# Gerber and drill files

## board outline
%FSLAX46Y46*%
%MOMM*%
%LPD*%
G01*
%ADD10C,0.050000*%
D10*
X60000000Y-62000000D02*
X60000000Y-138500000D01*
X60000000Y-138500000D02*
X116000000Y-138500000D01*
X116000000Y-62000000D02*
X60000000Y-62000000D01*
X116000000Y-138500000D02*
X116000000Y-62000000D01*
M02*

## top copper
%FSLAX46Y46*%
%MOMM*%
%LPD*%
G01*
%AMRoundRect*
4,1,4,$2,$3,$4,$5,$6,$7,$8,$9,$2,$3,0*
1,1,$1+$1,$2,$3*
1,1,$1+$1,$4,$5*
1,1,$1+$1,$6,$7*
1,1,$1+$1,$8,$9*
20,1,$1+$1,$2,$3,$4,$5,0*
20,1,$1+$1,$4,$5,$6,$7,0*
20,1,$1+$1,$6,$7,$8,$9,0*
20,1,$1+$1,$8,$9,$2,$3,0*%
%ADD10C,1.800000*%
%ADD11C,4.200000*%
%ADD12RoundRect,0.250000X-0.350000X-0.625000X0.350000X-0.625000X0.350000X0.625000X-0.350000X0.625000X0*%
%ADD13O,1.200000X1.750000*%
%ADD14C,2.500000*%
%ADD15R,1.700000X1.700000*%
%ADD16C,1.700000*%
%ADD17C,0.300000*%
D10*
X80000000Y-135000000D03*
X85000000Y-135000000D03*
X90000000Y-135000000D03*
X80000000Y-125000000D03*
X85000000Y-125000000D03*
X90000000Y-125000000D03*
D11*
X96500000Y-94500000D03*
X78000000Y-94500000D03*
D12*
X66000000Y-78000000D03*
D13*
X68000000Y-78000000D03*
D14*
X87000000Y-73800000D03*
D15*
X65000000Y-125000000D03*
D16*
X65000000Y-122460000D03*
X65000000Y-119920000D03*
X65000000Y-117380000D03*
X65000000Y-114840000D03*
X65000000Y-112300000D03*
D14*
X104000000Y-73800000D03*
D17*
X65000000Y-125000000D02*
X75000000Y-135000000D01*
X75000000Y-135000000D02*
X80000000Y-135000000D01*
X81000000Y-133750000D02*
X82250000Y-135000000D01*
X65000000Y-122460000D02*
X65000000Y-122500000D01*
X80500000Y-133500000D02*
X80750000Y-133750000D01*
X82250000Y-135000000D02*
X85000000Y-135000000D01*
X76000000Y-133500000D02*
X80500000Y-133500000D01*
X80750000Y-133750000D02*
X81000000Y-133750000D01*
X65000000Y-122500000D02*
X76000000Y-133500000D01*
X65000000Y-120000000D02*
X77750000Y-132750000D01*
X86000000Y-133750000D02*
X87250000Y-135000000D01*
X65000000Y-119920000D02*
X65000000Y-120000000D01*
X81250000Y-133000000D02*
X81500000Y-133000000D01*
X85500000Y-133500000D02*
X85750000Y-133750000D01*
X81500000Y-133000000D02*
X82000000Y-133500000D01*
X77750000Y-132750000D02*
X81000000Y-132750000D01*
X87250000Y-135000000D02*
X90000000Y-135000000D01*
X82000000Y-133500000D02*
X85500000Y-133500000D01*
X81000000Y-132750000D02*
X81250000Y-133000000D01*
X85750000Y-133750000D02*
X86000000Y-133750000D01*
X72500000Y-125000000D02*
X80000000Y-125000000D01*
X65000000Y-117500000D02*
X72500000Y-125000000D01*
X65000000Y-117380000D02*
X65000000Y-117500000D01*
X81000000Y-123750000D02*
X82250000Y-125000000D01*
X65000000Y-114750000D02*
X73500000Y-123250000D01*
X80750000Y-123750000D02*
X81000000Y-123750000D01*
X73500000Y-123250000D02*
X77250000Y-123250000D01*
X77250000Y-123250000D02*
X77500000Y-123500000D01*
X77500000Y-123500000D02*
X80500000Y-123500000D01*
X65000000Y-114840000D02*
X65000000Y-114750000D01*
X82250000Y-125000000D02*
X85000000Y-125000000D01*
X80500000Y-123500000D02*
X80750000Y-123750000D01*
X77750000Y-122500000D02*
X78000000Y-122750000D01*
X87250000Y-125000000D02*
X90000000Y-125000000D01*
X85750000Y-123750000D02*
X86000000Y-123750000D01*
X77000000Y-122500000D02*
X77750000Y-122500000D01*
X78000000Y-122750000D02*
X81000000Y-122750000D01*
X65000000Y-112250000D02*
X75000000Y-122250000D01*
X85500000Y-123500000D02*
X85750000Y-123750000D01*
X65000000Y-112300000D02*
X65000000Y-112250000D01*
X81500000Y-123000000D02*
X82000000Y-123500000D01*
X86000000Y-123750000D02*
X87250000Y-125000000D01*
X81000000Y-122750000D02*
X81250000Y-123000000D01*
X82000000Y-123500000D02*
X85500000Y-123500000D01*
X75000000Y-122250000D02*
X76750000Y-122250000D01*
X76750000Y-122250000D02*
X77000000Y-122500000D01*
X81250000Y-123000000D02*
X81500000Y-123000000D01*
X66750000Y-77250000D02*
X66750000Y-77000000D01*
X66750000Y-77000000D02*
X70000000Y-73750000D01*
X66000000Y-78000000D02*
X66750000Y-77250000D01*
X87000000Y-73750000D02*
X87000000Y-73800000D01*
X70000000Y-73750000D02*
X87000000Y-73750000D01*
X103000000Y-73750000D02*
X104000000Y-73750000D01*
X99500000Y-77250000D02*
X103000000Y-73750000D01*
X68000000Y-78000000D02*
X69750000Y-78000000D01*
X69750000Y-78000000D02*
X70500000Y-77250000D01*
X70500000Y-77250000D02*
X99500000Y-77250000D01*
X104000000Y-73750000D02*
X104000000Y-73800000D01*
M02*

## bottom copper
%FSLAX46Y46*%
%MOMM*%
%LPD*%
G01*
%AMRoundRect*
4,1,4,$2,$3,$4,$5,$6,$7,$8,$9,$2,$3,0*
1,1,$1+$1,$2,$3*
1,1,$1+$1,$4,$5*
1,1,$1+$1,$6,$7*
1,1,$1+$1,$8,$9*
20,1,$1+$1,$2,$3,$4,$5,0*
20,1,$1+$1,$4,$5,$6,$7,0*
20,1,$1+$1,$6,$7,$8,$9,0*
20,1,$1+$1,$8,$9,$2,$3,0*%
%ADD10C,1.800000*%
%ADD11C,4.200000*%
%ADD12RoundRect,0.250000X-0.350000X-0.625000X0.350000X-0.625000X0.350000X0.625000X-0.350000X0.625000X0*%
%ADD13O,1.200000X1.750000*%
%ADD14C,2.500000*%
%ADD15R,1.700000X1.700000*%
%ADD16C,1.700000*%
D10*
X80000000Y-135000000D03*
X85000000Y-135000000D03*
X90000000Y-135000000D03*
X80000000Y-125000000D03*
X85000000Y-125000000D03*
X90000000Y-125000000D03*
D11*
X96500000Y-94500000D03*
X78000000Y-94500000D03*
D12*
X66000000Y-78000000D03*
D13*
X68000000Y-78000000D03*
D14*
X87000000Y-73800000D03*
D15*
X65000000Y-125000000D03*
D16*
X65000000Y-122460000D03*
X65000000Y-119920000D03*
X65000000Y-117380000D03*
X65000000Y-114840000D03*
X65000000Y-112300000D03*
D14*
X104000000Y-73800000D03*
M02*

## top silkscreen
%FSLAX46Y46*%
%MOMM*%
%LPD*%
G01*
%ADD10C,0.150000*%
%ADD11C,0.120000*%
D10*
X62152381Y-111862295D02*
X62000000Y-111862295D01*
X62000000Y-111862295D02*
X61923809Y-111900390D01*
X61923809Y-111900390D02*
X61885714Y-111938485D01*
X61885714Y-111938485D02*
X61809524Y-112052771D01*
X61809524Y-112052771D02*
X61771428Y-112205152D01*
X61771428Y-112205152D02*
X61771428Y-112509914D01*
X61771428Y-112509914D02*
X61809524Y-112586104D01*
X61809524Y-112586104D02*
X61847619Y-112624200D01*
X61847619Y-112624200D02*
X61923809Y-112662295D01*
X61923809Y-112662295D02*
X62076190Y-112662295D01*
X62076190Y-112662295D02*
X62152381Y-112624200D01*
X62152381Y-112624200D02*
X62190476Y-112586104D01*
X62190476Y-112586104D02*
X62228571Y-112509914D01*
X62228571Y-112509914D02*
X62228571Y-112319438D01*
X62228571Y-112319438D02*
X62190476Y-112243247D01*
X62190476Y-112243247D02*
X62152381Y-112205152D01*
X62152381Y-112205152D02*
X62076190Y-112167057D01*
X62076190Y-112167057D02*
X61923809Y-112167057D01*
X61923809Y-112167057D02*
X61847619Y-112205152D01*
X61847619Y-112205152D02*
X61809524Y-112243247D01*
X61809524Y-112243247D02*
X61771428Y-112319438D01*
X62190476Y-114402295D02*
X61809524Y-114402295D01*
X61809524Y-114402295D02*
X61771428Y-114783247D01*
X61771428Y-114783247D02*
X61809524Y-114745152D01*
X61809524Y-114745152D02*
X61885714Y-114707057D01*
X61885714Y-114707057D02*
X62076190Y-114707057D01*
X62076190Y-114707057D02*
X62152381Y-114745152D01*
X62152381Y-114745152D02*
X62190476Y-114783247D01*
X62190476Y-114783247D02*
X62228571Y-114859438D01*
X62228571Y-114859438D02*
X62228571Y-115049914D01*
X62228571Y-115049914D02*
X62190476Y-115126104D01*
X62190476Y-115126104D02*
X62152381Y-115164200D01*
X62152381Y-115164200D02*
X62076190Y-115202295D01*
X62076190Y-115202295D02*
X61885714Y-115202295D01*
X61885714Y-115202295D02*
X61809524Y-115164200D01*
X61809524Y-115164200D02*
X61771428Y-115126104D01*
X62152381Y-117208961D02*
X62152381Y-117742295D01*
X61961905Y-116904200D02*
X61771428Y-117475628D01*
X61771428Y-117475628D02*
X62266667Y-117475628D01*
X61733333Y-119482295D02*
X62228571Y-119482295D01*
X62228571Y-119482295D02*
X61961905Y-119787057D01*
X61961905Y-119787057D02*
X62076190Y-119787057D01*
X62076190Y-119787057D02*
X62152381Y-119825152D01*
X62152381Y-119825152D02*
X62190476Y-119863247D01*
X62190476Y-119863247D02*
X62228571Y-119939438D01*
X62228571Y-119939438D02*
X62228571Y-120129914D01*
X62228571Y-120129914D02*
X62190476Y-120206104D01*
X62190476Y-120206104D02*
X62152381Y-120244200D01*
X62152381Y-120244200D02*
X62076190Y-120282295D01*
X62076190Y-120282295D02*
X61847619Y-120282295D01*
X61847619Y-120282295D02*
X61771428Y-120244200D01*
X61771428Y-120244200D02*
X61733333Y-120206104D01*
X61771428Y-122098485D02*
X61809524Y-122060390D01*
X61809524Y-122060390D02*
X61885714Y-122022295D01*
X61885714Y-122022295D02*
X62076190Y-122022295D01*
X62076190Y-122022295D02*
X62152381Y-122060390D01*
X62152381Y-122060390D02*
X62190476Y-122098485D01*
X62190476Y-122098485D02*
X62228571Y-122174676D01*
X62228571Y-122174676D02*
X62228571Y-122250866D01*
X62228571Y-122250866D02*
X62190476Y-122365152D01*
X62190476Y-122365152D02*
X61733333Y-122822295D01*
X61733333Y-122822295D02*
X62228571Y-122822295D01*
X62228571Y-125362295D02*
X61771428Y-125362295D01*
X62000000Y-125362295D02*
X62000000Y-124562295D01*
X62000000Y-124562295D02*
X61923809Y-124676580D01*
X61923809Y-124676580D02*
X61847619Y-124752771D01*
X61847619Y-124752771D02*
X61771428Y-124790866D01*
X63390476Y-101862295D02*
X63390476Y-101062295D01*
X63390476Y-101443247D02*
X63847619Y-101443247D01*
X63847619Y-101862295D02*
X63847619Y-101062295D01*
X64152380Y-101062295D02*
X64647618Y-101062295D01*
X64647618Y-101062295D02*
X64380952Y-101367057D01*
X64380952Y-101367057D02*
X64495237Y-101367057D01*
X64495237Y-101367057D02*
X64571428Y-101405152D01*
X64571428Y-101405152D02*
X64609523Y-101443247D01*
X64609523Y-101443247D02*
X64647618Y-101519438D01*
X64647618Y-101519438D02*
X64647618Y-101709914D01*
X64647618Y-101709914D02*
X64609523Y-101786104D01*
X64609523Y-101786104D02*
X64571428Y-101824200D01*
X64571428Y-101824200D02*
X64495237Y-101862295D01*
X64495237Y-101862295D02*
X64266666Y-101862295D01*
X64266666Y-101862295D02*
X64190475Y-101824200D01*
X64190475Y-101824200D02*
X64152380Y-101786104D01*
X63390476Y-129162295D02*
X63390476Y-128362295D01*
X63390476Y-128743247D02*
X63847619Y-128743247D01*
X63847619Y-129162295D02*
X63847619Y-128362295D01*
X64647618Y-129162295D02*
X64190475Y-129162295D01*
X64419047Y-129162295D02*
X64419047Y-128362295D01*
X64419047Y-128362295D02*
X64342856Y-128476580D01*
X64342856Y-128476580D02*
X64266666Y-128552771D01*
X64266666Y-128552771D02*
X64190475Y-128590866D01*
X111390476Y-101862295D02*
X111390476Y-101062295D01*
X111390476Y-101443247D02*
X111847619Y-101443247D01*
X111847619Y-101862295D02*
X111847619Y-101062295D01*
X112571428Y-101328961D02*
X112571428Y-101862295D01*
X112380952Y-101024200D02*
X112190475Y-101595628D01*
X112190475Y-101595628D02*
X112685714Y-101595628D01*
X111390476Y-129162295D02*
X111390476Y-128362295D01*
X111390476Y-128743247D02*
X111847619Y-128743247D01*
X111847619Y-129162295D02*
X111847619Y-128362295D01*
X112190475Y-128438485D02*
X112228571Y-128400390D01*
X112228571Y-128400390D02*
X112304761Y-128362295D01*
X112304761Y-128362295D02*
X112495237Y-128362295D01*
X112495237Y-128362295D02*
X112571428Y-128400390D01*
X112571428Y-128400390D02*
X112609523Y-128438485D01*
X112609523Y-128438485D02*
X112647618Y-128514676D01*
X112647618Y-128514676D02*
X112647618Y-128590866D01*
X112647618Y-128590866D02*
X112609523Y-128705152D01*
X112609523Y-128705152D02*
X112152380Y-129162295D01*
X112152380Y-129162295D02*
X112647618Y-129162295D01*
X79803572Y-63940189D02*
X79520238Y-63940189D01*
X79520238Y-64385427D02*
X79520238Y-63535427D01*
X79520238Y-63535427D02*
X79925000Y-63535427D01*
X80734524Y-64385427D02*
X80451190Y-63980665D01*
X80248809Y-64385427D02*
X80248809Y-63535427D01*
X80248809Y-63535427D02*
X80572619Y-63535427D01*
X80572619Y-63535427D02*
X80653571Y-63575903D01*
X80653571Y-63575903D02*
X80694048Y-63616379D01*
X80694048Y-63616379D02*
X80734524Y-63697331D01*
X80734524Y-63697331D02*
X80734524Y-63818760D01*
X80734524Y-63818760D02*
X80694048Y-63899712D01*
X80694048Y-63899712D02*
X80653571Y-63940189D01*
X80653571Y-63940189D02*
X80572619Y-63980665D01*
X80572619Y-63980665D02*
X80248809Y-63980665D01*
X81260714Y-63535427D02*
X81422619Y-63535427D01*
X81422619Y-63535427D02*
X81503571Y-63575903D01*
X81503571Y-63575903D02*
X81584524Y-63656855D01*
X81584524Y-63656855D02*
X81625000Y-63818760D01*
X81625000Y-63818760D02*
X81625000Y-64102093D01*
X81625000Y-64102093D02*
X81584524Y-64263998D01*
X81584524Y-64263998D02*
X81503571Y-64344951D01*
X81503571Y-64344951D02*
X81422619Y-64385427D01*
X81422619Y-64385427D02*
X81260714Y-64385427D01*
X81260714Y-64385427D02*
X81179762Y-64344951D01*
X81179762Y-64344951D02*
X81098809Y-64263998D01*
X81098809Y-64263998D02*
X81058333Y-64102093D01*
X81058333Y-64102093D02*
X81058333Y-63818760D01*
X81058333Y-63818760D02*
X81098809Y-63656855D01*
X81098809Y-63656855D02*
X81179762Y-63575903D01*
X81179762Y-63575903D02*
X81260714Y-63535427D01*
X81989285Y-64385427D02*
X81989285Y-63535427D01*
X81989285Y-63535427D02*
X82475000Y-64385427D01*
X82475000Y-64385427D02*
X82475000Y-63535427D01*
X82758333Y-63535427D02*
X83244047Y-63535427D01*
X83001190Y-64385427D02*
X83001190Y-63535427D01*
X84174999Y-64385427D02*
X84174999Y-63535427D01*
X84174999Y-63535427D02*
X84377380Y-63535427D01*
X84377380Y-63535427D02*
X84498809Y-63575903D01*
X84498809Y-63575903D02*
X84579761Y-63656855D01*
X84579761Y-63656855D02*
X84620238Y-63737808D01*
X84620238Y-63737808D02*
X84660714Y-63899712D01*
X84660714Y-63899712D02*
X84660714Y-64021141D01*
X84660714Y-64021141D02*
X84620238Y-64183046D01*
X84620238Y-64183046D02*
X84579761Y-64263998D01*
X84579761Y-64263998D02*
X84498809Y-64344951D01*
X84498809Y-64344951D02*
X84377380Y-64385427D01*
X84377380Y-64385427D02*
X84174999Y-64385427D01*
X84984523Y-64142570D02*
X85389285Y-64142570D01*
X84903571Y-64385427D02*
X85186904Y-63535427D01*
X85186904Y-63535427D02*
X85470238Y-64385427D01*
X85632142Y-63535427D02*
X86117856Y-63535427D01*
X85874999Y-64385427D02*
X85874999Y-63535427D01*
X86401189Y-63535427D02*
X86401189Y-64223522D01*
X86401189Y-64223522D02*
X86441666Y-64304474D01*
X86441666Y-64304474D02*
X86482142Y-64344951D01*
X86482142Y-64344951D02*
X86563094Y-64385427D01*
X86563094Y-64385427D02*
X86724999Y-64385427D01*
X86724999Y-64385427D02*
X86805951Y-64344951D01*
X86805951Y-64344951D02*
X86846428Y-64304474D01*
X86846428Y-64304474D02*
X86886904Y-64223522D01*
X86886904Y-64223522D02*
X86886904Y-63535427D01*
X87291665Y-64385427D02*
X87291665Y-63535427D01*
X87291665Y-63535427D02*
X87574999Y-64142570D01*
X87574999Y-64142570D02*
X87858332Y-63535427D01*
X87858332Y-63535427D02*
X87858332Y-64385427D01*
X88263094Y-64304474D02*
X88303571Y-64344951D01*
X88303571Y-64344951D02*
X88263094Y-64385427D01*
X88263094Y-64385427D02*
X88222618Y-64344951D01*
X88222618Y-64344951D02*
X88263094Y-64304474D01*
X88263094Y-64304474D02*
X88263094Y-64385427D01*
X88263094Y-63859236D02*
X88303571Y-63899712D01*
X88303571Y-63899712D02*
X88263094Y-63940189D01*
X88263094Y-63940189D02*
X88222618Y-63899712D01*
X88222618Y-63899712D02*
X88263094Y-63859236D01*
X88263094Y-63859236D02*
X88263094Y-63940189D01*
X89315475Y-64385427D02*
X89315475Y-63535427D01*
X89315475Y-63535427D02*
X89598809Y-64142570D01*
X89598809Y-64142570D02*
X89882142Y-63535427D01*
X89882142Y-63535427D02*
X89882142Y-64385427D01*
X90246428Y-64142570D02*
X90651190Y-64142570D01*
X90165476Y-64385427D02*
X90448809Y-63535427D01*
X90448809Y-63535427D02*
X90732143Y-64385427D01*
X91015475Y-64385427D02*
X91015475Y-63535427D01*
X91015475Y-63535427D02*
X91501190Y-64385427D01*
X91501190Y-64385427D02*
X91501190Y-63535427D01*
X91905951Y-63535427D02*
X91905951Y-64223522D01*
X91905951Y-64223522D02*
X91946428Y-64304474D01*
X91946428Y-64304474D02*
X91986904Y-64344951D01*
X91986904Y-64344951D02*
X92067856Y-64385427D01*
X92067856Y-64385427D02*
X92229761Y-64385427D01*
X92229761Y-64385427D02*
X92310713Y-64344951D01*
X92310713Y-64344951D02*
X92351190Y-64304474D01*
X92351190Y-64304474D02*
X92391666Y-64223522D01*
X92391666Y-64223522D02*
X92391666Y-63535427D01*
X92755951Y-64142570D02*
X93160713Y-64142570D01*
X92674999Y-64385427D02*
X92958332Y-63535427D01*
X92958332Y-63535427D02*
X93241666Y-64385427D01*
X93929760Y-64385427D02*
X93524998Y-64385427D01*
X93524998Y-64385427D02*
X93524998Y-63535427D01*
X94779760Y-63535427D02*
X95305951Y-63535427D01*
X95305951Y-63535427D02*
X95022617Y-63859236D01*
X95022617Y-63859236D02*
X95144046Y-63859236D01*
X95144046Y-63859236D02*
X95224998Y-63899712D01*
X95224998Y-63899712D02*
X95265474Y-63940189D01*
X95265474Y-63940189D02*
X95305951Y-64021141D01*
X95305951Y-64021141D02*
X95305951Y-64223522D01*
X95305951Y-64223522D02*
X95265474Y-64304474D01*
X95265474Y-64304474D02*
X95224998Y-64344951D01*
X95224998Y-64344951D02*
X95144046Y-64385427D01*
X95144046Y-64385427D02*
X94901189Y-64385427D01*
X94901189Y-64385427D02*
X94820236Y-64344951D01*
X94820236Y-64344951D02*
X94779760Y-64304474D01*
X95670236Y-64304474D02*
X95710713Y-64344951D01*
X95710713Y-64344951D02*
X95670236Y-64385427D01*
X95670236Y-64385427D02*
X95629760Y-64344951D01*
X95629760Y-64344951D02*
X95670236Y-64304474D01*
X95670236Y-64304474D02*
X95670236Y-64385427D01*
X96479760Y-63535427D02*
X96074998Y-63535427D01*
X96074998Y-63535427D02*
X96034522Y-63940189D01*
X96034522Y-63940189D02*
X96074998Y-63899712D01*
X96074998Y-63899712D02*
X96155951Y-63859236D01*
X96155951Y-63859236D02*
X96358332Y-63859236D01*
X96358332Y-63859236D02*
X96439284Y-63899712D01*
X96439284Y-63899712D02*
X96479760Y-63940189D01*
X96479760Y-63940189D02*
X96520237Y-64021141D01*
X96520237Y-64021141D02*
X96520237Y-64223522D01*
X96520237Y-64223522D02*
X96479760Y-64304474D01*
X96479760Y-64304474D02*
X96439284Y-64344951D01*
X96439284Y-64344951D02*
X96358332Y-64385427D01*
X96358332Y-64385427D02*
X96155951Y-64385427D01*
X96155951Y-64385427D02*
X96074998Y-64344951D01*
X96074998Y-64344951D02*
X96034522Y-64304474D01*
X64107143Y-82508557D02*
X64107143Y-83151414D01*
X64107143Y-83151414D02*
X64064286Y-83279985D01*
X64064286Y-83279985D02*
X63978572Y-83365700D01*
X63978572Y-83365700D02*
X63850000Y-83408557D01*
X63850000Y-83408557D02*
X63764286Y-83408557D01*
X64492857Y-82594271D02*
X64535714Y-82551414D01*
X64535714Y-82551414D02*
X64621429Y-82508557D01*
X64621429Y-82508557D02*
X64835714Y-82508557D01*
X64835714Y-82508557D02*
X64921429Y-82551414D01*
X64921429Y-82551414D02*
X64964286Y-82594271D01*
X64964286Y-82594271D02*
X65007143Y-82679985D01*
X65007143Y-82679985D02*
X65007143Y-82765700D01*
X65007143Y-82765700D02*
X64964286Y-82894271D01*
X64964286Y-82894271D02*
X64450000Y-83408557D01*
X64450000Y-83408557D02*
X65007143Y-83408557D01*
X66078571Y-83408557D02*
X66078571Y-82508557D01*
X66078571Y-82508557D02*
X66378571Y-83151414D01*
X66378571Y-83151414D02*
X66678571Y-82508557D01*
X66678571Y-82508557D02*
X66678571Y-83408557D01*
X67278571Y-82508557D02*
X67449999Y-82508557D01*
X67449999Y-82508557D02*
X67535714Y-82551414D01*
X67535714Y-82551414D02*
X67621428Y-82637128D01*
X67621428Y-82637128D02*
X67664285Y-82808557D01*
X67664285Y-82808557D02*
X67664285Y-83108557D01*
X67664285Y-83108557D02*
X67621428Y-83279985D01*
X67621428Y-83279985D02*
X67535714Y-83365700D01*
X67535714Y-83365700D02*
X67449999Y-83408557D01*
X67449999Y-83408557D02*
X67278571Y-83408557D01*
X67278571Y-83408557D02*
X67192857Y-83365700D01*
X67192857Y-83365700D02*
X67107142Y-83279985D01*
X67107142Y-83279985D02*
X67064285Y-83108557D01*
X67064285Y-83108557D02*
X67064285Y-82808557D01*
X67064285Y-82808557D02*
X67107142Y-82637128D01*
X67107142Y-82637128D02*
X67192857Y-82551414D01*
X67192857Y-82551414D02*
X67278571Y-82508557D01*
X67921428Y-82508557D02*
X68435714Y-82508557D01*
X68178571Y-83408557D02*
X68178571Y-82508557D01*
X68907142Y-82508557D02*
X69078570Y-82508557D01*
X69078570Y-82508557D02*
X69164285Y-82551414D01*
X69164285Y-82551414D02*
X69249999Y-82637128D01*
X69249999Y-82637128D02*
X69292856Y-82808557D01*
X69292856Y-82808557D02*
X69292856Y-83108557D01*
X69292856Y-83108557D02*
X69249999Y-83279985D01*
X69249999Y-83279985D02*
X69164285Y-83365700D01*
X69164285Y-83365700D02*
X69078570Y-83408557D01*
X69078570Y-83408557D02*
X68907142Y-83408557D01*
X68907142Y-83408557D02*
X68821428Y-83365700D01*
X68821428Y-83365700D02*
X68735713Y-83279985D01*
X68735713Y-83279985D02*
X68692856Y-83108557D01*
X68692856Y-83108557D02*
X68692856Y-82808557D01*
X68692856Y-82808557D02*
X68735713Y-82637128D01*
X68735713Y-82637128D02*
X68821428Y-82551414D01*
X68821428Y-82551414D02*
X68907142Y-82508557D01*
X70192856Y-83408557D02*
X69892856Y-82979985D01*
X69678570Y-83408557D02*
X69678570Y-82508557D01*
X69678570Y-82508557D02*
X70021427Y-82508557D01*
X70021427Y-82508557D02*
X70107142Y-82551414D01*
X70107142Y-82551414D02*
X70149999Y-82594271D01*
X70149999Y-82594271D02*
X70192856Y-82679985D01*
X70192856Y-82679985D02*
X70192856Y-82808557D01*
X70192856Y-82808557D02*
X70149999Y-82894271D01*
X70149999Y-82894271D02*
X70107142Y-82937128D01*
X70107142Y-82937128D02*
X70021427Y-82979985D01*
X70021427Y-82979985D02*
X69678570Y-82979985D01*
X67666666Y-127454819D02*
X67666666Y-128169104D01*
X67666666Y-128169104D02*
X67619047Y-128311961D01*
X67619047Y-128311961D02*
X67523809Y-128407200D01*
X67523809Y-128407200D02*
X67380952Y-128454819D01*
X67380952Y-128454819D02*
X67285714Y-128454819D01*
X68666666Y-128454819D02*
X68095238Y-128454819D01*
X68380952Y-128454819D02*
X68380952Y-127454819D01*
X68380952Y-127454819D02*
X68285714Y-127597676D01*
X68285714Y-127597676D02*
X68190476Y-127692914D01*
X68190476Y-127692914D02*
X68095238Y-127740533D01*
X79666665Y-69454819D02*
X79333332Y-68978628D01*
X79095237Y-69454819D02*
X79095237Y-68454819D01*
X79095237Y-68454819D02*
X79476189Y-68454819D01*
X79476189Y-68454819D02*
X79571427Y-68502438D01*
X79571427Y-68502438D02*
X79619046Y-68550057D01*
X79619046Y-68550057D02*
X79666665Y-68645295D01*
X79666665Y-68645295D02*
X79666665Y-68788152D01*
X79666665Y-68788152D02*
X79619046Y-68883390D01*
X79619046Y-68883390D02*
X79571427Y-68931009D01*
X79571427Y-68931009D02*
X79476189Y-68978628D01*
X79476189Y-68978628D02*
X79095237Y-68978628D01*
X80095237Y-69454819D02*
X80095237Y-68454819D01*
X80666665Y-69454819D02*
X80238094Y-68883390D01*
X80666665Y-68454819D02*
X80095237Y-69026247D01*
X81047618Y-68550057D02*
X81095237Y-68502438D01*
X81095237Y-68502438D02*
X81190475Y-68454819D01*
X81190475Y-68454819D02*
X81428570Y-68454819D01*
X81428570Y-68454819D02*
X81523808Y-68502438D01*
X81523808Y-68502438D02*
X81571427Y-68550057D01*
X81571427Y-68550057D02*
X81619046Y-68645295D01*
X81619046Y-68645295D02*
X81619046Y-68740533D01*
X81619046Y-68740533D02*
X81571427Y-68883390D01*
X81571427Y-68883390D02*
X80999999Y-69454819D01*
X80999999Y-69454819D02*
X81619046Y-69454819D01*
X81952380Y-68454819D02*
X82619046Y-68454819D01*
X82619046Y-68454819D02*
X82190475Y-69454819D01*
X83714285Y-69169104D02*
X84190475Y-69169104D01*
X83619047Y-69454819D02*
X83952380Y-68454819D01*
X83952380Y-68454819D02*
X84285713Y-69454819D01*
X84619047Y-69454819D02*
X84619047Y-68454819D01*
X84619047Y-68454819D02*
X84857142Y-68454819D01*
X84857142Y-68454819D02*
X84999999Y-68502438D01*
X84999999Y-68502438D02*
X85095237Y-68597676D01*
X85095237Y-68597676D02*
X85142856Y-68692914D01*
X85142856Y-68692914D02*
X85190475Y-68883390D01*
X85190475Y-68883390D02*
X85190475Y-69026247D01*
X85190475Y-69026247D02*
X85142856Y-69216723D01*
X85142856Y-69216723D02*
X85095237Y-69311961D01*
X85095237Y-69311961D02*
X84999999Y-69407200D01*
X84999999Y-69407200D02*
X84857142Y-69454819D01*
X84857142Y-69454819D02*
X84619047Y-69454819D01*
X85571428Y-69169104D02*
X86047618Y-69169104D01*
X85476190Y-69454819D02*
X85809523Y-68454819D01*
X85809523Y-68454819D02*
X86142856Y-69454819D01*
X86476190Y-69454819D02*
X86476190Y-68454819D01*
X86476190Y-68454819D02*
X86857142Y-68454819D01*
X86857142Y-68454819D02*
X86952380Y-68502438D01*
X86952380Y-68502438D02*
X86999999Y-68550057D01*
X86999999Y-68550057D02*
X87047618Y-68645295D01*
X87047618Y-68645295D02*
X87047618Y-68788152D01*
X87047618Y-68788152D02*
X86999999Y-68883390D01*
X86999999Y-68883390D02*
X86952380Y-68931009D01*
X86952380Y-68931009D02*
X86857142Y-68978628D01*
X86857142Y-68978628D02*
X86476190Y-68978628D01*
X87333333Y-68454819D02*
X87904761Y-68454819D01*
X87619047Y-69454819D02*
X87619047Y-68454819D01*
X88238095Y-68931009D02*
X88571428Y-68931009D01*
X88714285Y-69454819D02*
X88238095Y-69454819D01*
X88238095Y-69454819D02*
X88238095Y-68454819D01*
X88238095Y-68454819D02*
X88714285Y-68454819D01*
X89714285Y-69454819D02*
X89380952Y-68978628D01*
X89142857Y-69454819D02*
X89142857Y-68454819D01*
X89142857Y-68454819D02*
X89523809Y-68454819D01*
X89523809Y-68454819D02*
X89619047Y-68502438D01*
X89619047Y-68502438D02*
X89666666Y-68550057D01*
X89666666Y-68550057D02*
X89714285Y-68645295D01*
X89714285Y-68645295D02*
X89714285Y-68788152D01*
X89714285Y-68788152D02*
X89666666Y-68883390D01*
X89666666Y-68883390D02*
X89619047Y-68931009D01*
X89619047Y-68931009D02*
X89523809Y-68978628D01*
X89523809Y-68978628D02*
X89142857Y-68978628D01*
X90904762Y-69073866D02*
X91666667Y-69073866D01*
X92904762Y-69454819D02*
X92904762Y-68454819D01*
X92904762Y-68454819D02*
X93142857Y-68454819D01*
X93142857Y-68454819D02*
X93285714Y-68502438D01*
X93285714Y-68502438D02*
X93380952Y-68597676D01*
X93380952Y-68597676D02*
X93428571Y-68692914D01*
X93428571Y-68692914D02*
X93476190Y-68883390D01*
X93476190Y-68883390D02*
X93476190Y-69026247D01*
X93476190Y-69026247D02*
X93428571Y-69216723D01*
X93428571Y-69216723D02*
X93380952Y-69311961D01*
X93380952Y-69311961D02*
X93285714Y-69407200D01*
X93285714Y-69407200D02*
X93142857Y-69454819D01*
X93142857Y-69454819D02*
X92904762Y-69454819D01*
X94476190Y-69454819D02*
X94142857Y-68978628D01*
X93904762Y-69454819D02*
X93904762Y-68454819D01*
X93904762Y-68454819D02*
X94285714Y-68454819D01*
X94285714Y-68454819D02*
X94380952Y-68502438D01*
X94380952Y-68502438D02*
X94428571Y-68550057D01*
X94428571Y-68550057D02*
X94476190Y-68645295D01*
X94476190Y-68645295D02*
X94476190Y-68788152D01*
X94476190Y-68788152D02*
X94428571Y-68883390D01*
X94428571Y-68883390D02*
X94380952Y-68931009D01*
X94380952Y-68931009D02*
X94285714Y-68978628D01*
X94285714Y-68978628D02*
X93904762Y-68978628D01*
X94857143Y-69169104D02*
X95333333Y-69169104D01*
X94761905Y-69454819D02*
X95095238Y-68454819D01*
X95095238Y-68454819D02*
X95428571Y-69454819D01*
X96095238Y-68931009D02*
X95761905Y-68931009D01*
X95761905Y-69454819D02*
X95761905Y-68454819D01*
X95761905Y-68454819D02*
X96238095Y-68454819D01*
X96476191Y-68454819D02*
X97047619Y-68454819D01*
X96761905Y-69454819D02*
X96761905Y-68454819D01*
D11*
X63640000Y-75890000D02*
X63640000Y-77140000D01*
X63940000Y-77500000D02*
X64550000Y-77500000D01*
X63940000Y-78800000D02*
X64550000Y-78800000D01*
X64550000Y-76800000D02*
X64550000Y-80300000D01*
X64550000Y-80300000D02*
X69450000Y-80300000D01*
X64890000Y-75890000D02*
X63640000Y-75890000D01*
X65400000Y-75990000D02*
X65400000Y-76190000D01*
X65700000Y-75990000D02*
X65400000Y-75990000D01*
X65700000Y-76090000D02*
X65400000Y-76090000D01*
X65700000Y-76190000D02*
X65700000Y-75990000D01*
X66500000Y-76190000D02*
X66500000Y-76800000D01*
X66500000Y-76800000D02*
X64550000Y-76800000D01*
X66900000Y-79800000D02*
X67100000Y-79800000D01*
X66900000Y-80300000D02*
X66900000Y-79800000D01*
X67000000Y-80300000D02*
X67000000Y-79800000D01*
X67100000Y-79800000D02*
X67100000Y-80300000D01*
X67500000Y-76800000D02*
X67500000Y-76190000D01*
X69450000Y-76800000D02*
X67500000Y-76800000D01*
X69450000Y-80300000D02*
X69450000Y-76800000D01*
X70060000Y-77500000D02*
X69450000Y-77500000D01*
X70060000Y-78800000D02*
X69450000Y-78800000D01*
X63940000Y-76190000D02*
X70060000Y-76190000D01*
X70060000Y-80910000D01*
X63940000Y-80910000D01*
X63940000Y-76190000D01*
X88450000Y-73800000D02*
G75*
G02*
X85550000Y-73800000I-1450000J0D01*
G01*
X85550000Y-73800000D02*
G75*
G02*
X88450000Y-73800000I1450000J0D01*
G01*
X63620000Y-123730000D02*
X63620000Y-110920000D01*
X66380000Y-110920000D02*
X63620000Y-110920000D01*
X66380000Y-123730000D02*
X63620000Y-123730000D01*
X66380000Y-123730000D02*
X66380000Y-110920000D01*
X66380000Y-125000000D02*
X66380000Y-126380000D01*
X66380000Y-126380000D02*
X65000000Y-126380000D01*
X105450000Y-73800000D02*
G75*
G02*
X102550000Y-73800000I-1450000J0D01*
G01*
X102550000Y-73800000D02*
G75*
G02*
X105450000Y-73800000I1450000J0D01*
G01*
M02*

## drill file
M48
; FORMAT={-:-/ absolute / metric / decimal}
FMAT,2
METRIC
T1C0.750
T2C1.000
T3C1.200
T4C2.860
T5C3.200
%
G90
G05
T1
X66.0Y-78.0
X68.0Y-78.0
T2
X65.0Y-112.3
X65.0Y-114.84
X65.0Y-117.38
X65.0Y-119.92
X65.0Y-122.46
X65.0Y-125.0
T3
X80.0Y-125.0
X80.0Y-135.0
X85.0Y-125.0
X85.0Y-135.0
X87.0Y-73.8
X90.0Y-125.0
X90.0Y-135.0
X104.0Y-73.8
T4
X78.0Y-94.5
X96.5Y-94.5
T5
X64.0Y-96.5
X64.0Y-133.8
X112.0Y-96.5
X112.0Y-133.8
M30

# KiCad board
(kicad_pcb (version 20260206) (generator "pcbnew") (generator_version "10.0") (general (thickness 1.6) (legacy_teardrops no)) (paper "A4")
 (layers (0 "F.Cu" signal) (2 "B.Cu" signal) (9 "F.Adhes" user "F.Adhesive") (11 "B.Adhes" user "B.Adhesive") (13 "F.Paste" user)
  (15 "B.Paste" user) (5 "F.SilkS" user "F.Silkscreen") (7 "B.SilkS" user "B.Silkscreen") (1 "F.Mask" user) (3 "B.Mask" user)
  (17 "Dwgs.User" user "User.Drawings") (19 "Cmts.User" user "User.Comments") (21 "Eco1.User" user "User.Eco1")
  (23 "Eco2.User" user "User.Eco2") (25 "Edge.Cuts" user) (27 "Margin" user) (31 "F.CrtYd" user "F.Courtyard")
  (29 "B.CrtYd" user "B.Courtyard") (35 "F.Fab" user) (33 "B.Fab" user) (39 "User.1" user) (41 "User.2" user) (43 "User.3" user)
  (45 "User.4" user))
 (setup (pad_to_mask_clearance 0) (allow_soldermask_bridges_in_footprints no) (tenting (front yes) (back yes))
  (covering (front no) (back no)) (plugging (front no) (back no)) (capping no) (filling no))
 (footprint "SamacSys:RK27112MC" (layer "F.Cu") (at 85 94.5 -90)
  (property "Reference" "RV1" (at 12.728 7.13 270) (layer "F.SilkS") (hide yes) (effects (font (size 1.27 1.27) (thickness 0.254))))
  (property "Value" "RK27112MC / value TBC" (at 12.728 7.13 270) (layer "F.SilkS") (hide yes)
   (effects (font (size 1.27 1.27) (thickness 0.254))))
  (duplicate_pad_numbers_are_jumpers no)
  (pad "1" thru_hole circle (at 40.5 5 270) (size 1.8 1.8) (drill 1.2) (layers "*.Cu" "*.Mask") (remove_unused_layers no) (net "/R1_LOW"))
  (pad "2" thru_hole circle (at 40.5 0 270) (size 1.8 1.8) (drill 1.2) (layers "*.Cu" "*.Mask") (remove_unused_layers no) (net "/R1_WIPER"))
  (pad "3" thru_hole circle (at 40.5 -5 270) (size 1.8 1.8) (drill 1.2) (layers "*.Cu" "*.Mask") (remove_unused_layers no) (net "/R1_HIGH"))
  (pad "4" thru_hole circle (at 30.5 5 270) (size 1.8 1.8) (drill 1.2) (layers "*.Cu" "*.Mask") (remove_unused_layers no) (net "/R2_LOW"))
  (pad "5" thru_hole circle (at 30.5 0 270) (size 1.8 1.8) (drill 1.2) (layers "*.Cu" "*.Mask") (remove_unused_layers no) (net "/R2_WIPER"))
  (pad "6" thru_hole circle (at 30.5 -5 270) (size 1.8 1.8) (drill 1.2) (layers "*.Cu" "*.Mask") (remove_unused_layers no) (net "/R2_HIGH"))
  (pad "7" thru_hole circle (at 0 -11.5 270) (size 4.2 4.2) (drill 2.86) (layers "*.Cu" "*.Mask") (remove_unused_layers no)
   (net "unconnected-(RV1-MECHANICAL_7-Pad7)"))
  (pad "8" thru_hole circle (at 0 7 270) (size 4.2 4.2) (drill 2.86) (layers "*.Cu" "*.Mask") (remove_unused_layers no)
   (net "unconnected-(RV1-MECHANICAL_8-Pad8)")))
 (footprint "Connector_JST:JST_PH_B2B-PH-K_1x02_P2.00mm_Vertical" (layer "F.Cu") (at 66 78)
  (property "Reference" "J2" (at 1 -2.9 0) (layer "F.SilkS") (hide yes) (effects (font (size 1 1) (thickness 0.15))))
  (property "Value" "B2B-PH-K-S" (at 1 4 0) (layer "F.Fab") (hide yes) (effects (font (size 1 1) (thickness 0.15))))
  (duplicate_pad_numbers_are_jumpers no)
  (fp_line (start -2.36 -2.11) (end -2.36 -0.86) (stroke (width 0.12) (type solid)) (layer "F.SilkS"))
  (fp_line (start -2.06 -0.5) (end -1.45 -0.5) (stroke (width 0.12) (type solid)) (layer "F.SilkS"))
  (fp_line (start -2.06 0.8) (end -1.45 0.8) (stroke (width 0.12) (type solid)) (layer "F.SilkS"))
  (fp_line (start -1.45 -1.2) (end -1.45 2.3) (stroke (width 0.12) (type solid)) (layer "F.SilkS"))
  (fp_line (start -1.45 2.3) (end 3.45 2.3) (stroke (width 0.12) (type solid)) (layer "F.SilkS"))
  (fp_line (start -1.11 -2.11) (end -2.36 -2.11) (stroke (width 0.12) (type solid)) (layer "F.SilkS"))
  (fp_line (start -0.6 -2.01) (end -0.6 -1.81) (stroke (width 0.12) (type solid)) (layer "F.SilkS"))
  (fp_line (start -0.3 -2.01) (end -0.6 -2.01) (stroke (width 0.12) (type solid)) (layer "F.SilkS"))
  (fp_line (start -0.3 -1.91) (end -0.6 -1.91) (stroke (width 0.12) (type solid)) (layer "F.SilkS"))
  (fp_line (start -0.3 -1.81) (end -0.3 -2.01) (stroke (width 0.12) (type solid)) (layer "F.SilkS"))
  (fp_line (start 0.5 -1.81) (end 0.5 -1.2) (stroke (width 0.12) (type solid)) (layer "F.SilkS"))
  (fp_line (start 0.5 -1.2) (end -1.45 -1.2) (stroke (width 0.12) (type solid)) (layer "F.SilkS"))
  (fp_line (start 0.9 1.8) (end 1.1 1.8) (stroke (width 0.12) (type solid)) (layer "F.SilkS"))
  (fp_line (start 0.9 2.3) (end 0.9 1.8) (stroke (width 0.12) (type solid)) (layer "F.SilkS"))
  (fp_line (start 1 2.3) (end 1 1.8) (stroke (width 0.12) (type solid)) (layer "F.SilkS"))
  (fp_line (start 1.1 1.8) (end 1.1 2.3) (stroke (width 0.12) (type solid)) (layer "F.SilkS"))
  (fp_line (start 1.5 -1.2) (end 1.5 -1.81) (stroke (width 0.12) (type solid)) (layer "F.SilkS"))
  (fp_line (start 3.45 -1.2) (end 1.5 -1.2) (stroke (width 0.12) (type solid)) (layer "F.SilkS"))
  (fp_line (start 3.45 2.3) (end 3.45 -1.2) (stroke (width 0.12) (type solid)) (layer "F.SilkS"))
  (fp_line (start 4.06 -0.5) (end 3.45 -0.5) (stroke (width 0.12) (type solid)) (layer "F.SilkS"))
  (fp_line (start 4.06 0.8) (end 3.45 0.8) (stroke (width 0.12) (type solid)) (layer "F.SilkS"))
  (fp_rect (start -2.06 -1.81) (end 4.06 2.91) (stroke (width 0.12) (type solid)) (fill no) (layer "F.SilkS"))
  (pad "1" thru_hole roundrect (at 0 0) (size 1.2 1.75) (drill 0.75) (layers "*.Cu" "*.Mask") (remove_unused_layers no)
   (roundrect_rratio 0.208333) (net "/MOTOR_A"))
  (pad "2" thru_hole oval (at 2 0) (size 1.2 1.75) (drill 0.75) (layers "*.Cu" "*.Mask") (remove_unused_layers no) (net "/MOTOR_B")))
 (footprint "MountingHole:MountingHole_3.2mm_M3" (layer "F.Cu") (at 112 133.8)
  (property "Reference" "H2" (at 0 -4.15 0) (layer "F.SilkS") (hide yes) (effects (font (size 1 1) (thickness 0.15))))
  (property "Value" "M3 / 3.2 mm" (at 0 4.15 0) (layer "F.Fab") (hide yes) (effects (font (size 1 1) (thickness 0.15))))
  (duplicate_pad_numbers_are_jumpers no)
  (pad "" np_thru_hole circle (at 0 0) (size 3.2 3.2) (drill 3.2) (layers "*.Cu" "*.Mask")))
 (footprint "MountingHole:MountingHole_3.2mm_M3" (layer "F.Cu") (at 64 96.5)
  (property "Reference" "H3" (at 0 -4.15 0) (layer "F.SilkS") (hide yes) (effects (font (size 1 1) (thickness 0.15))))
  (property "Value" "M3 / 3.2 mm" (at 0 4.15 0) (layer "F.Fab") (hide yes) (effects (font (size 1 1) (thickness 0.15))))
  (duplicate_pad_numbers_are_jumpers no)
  (pad "" np_thru_hole circle (at 0 0) (size 3.2 3.2) (drill 3.2) (layers "*.Cu" "*.Mask")))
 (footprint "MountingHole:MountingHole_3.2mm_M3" (layer "F.Cu") (at 64 133.8)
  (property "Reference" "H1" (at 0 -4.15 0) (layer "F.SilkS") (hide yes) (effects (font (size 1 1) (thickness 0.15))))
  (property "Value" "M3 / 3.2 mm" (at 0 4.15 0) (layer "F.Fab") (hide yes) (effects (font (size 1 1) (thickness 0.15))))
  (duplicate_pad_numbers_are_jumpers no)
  (pad "" np_thru_hole circle (at 0 0) (size 3.2 3.2) (drill 3.2) (layers "*.Cu" "*.Mask")))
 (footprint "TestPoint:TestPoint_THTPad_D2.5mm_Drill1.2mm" (layer "F.Cu") (at 87 73.8)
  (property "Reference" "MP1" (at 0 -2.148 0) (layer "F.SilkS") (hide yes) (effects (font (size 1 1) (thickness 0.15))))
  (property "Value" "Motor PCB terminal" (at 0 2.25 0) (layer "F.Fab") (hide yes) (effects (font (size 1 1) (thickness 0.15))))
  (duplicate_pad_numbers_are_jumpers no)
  (fp_circle (center 0 0) (end 0 1.45) (stroke (width 0.12) (type solid)) (fill no) (layer "F.SilkS"))
  (pad "1" thru_hole circle (at 0 0) (size 2.5 2.5) (drill 1.2) (layers "*.Cu" "*.Mask") (remove_unused_layers no) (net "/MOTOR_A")))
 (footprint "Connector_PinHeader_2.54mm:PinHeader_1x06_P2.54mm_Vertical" (layer "F.Cu") (at 65 125 180)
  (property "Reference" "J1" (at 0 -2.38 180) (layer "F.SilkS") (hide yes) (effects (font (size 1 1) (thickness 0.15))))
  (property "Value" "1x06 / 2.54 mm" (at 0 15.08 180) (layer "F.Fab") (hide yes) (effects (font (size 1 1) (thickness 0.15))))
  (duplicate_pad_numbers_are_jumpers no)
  (fp_line (start 1.38 1.27) (end 1.38 14.08) (stroke (width 0.12) (type solid)) (layer "F.SilkS"))
  (fp_line (start -1.38 14.08) (end 1.38 14.08) (stroke (width 0.12) (type solid)) (layer "F.SilkS"))
  (fp_line (start -1.38 1.27) (end 1.38 1.27) (stroke (width 0.12) (type solid)) (layer "F.SilkS"))
  (fp_line (start -1.38 1.27) (end -1.38 14.08) (stroke (width 0.12) (type solid)) (layer "F.SilkS"))
  (fp_line (start -1.38 0) (end -1.38 -1.38) (stroke (width 0.12) (type solid)) (layer "F.SilkS"))
  (fp_line (start -1.38 -1.38) (end 0 -1.38) (stroke (width 0.12) (type solid)) (layer "F.SilkS"))
  (pad "1" thru_hole rect (at 0 0 180) (size 1.7 1.7) (drill 1) (layers "*.Cu" "*.Mask") (remove_unused_layers no) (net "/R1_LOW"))
  (pad "2" thru_hole circle (at 0 2.54 180) (size 1.7 1.7) (drill 1) (layers "*.Cu" "*.Mask") (remove_unused_layers no) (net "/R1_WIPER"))
  (pad "3" thru_hole circle (at 0 5.08 180) (size 1.7 1.7) (drill 1) (layers "*.Cu" "*.Mask") (remove_unused_layers no) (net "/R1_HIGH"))
  (pad "4" thru_hole circle (at 0 7.62 180) (size 1.7 1.7) (drill 1) (layers "*.Cu" "*.Mask") (remove_unused_layers no) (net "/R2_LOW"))
  (pad "5" thru_hole circle (at 0 10.16 180) (size 1.7 1.7) (drill 1) (layers "*.Cu" "*.Mask") (remove_unused_layers no) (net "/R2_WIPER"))
  (pad "6" thru_hole circle (at 0 12.7 180) (size 1.7 1.7) (drill 1) (layers "*.Cu" "*.Mask") (remove_unused_layers no) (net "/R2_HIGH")))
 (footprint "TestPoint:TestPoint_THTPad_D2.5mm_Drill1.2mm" (layer "F.Cu") (at 104 73.8)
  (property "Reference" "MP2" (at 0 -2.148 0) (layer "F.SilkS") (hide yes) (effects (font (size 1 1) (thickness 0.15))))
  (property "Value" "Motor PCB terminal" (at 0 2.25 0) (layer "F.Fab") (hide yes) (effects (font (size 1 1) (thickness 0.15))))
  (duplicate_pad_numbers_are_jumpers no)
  (fp_circle (center 0 0) (end 0 1.45) (stroke (width 0.12) (type solid)) (fill no) (layer "F.SilkS"))
  (pad "1" thru_hole circle (at 0 0) (size 2.5 2.5) (drill 1.2) (layers "*.Cu" "*.Mask") (remove_unused_layers no) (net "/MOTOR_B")))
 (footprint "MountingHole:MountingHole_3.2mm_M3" (layer "F.Cu") (at 112 96.5)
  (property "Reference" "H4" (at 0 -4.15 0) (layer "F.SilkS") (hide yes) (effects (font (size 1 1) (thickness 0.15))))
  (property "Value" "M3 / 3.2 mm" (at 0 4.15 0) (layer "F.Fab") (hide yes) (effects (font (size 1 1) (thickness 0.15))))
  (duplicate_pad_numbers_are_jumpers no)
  (pad "" np_thru_hole circle (at 0 0) (size 3.2 3.2) (drill 3.2) (layers "*.Cu" "*.Mask")))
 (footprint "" (layer "F.Cu") (at 85 140)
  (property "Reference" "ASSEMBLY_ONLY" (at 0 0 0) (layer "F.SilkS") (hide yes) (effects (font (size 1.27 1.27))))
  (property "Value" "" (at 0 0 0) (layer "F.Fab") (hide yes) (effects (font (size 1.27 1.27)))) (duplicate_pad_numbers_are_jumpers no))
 (gr_line (start 60 62) (end 60 138.5) (stroke (width 0.05) (type default)) (layer "Edge.Cuts"))
 (gr_line (start 60 138.5) (end 116 138.5) (stroke (width 0.05) (type default)) (layer "Edge.Cuts"))
 (gr_line (start 116 62) (end 60 62) (stroke (width 0.05) (type default)) (layer "Edge.Cuts"))
 (gr_line (start 116 138.5) (end 116 62) (stroke (width 0.05) (type default)) (layer "Edge.Cuts"))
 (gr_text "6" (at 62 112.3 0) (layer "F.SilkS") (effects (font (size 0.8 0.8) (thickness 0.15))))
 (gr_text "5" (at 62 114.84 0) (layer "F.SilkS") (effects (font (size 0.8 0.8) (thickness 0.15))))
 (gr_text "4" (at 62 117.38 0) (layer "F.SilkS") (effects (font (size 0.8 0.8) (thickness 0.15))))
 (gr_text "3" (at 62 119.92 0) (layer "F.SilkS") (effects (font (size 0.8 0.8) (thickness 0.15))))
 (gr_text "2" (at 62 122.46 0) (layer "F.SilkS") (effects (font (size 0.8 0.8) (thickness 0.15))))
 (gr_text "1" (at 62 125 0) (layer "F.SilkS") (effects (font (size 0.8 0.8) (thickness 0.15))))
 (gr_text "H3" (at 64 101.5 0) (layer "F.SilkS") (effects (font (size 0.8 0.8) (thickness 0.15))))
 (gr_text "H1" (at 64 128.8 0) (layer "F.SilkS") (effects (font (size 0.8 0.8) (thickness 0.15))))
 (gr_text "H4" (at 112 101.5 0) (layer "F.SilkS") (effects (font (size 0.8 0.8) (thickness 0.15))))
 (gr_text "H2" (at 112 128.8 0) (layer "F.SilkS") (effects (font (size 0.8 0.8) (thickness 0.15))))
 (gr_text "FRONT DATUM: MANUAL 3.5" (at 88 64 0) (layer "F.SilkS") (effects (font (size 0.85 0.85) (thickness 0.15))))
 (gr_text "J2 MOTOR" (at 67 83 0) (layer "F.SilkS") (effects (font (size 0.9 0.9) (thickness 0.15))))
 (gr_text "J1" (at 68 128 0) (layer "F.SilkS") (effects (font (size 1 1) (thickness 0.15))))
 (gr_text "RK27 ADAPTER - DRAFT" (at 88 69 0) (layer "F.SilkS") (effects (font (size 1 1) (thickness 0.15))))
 (segment (start 65 125) (end 75 135) (width 0.3) (layer "F.Cu") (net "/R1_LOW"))
 (segment (start 75 135) (end 80 135) (width 0.3) (layer "F.Cu") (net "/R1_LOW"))
 (segment (start 81 133.75) (end 82.25 135) (width 0.3) (layer "F.Cu") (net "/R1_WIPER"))
 (segment (start 65 122.46) (end 65 122.5) (width 0.3) (layer "F.Cu") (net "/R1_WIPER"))
 (segment (start 80.5 133.5) (end 80.75 133.75) (width 0.3) (layer "F.Cu") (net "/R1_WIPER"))
 (segment (start 82.25 135) (end 85 135) (width 0.3) (layer "F.Cu") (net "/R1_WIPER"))
 (segment (start 76 133.5) (end 80.5 133.5) (width 0.3) (layer "F.Cu") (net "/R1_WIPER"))
 (segment (start 80.75 133.75) (end 81 133.75) (width 0.3) (layer "F.Cu") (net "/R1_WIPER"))
 (segment (start 65 122.5) (end 76 133.5) (width 0.3) (layer "F.Cu") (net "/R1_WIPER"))
 (segment (start 65 120) (end 77.75 132.75) (width 0.3) (layer "F.Cu") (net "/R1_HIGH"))
 (segment (start 86 133.75) (end 87.25 135) (width 0.3) (layer "F.Cu") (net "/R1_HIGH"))
 (segment (start 65 119.92) (end 65 120) (width 0.3) (layer "F.Cu") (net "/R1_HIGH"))
 (segment (start 81.25 133) (end 81.5 133) (width 0.3) (layer "F.Cu") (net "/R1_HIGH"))
 (segment (start 85.5 133.5) (end 85.75 133.75) (width 0.3) (layer "F.Cu") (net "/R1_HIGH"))
 (segment (start 81.5 133) (end 82 133.5) (width 0.3) (layer "F.Cu") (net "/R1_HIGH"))
 (segment (start 77.75 132.75) (end 81 132.75) (width 0.3) (layer "F.Cu") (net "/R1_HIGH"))
 (segment (start 87.25 135) (end 90 135) (width 0.3) (layer "F.Cu") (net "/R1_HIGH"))
 (segment (start 82 133.5) (end 85.5 133.5) (width 0.3) (layer "F.Cu") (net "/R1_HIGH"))
 (segment (start 81 132.75) (end 81.25 133) (width 0.3) (layer "F.Cu") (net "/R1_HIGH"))
 (segment (start 85.75 133.75) (end 86 133.75) (width 0.3) (layer "F.Cu") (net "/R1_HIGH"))
 (segment (start 72.5 125) (end 80 125) (width 0.3) (layer "F.Cu") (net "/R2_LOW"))
 (segment (start 65 117.5) (end 72.5 125) (width 0.3) (layer "F.Cu") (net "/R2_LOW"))
 (segment (start 65 117.38) (end 65 117.5) (width 0.3) (layer "F.Cu") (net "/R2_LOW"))
 (segment (start 81 123.75) (end 82.25 125) (width 0.3) (layer "F.Cu") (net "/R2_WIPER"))
 (segment (start 65 114.75) (end 73.5 123.25) (width 0.3) (layer "F.Cu") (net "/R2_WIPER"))
 (segment (start 80.75 123.75) (end 81 123.75) (width 0.3) (layer "F.Cu") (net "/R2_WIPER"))
 (segment (start 73.5 123.25) (end 77.25 123.25) (width 0.3) (layer "F.Cu") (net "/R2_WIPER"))
 (segment (start 77.25 123.25) (end 77.5 123.5) (width 0.3) (layer "F.Cu") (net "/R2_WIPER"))
 (segment (start 77.5 123.5) (end 80.5 123.5) (width 0.3) (layer "F.Cu") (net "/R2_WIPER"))
 (segment (start 65 114.84) (end 65 114.75) (width 0.3) (layer "F.Cu") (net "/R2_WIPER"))
 (segment (start 82.25 125) (end 85 125) (width 0.3) (layer "F.Cu") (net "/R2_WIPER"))
 (segment (start 80.5 123.5) (end 80.75 123.75) (width 0.3) (layer "F.Cu") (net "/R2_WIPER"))
 (segment (start 77.75 122.5) (end 78 122.75) (width 0.3) (layer "F.Cu") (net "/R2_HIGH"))
 (segment (start 87.25 125) (end 90 125) (width 0.3) (layer "F.Cu") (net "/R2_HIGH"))
 (segment (start 85.75 123.75) (end 86 123.75) (width 0.3) (layer "F.Cu") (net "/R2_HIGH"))
 (segment (start 77 122.5) (end 77.75 122.5) (width 0.3) (layer "F.Cu") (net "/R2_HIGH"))
 (segment (start 78 122.75) (end 81 122.75) (width 0.3) (layer "F.Cu") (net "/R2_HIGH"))
 (segment (start 65 112.25) (end 75 122.25) (width 0.3) (layer "F.Cu") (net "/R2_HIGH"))
 (segment (start 85.5 123.5) (end 85.75 123.75) (width 0.3) (layer "F.Cu") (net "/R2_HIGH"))
 (segment (start 65 112.3) (end 65 112.25) (width 0.3) (layer "F.Cu") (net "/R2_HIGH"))
 (segment (start 81.5 123) (end 82 123.5) (width 0.3) (layer "F.Cu") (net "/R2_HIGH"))
 (segment (start 86 123.75) (end 87.25 125) (width 0.3) (layer "F.Cu") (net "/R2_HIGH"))
 (segment (start 81 122.75) (end 81.25 123) (width 0.3) (layer "F.Cu") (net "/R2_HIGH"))
 (segment (start 82 123.5) (end 85.5 123.5) (width 0.3) (layer "F.Cu") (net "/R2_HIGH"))
 (segment (start 75 122.25) (end 76.75 122.25) (width 0.3) (layer "F.Cu") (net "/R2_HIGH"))
 (segment (start 76.75 122.25) (end 77 122.5) (width 0.3) (layer "F.Cu") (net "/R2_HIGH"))
 (segment (start 81.25 123) (end 81.5 123) (width 0.3) (layer "F.Cu") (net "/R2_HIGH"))
 (segment (start 66.75 77.25) (end 66.75 77) (width 0.3) (layer "F.Cu") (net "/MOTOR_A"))
 (segment (start 66.75 77) (end 70 73.75) (width 0.3) (layer "F.Cu") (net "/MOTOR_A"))
 (segment (start 66 78) (end 66.75 77.25) (width 0.3) (layer "F.Cu") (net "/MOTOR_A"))
 (segment (start 87 73.75) (end 87 73.8) (width 0.3) (layer "F.Cu") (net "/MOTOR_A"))
 (segment (start 70 73.75) (end 87 73.75) (width 0.3) (layer "F.Cu") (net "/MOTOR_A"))
 (segment (start 103 73.75) (end 104 73.75) (width 0.3) (layer "F.Cu") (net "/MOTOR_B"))
 (segment (start 99.5 77.25) (end 103 73.75) (width 0.3) (layer "F.Cu") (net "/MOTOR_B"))
 (segment (start 68 78) (end 69.75 78) (width 0.3) (layer "F.Cu") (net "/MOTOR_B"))
 (segment (start 69.75 78) (end 70.5 77.25) (width 0.3) (layer "F.Cu") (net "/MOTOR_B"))
 (segment (start 70.5 77.25) (end 99.5 77.25) (width 0.3) (layer "F.Cu") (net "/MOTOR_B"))
 (segment (start 104 73.75) (end 104 73.8) (width 0.3) (layer "F.Cu") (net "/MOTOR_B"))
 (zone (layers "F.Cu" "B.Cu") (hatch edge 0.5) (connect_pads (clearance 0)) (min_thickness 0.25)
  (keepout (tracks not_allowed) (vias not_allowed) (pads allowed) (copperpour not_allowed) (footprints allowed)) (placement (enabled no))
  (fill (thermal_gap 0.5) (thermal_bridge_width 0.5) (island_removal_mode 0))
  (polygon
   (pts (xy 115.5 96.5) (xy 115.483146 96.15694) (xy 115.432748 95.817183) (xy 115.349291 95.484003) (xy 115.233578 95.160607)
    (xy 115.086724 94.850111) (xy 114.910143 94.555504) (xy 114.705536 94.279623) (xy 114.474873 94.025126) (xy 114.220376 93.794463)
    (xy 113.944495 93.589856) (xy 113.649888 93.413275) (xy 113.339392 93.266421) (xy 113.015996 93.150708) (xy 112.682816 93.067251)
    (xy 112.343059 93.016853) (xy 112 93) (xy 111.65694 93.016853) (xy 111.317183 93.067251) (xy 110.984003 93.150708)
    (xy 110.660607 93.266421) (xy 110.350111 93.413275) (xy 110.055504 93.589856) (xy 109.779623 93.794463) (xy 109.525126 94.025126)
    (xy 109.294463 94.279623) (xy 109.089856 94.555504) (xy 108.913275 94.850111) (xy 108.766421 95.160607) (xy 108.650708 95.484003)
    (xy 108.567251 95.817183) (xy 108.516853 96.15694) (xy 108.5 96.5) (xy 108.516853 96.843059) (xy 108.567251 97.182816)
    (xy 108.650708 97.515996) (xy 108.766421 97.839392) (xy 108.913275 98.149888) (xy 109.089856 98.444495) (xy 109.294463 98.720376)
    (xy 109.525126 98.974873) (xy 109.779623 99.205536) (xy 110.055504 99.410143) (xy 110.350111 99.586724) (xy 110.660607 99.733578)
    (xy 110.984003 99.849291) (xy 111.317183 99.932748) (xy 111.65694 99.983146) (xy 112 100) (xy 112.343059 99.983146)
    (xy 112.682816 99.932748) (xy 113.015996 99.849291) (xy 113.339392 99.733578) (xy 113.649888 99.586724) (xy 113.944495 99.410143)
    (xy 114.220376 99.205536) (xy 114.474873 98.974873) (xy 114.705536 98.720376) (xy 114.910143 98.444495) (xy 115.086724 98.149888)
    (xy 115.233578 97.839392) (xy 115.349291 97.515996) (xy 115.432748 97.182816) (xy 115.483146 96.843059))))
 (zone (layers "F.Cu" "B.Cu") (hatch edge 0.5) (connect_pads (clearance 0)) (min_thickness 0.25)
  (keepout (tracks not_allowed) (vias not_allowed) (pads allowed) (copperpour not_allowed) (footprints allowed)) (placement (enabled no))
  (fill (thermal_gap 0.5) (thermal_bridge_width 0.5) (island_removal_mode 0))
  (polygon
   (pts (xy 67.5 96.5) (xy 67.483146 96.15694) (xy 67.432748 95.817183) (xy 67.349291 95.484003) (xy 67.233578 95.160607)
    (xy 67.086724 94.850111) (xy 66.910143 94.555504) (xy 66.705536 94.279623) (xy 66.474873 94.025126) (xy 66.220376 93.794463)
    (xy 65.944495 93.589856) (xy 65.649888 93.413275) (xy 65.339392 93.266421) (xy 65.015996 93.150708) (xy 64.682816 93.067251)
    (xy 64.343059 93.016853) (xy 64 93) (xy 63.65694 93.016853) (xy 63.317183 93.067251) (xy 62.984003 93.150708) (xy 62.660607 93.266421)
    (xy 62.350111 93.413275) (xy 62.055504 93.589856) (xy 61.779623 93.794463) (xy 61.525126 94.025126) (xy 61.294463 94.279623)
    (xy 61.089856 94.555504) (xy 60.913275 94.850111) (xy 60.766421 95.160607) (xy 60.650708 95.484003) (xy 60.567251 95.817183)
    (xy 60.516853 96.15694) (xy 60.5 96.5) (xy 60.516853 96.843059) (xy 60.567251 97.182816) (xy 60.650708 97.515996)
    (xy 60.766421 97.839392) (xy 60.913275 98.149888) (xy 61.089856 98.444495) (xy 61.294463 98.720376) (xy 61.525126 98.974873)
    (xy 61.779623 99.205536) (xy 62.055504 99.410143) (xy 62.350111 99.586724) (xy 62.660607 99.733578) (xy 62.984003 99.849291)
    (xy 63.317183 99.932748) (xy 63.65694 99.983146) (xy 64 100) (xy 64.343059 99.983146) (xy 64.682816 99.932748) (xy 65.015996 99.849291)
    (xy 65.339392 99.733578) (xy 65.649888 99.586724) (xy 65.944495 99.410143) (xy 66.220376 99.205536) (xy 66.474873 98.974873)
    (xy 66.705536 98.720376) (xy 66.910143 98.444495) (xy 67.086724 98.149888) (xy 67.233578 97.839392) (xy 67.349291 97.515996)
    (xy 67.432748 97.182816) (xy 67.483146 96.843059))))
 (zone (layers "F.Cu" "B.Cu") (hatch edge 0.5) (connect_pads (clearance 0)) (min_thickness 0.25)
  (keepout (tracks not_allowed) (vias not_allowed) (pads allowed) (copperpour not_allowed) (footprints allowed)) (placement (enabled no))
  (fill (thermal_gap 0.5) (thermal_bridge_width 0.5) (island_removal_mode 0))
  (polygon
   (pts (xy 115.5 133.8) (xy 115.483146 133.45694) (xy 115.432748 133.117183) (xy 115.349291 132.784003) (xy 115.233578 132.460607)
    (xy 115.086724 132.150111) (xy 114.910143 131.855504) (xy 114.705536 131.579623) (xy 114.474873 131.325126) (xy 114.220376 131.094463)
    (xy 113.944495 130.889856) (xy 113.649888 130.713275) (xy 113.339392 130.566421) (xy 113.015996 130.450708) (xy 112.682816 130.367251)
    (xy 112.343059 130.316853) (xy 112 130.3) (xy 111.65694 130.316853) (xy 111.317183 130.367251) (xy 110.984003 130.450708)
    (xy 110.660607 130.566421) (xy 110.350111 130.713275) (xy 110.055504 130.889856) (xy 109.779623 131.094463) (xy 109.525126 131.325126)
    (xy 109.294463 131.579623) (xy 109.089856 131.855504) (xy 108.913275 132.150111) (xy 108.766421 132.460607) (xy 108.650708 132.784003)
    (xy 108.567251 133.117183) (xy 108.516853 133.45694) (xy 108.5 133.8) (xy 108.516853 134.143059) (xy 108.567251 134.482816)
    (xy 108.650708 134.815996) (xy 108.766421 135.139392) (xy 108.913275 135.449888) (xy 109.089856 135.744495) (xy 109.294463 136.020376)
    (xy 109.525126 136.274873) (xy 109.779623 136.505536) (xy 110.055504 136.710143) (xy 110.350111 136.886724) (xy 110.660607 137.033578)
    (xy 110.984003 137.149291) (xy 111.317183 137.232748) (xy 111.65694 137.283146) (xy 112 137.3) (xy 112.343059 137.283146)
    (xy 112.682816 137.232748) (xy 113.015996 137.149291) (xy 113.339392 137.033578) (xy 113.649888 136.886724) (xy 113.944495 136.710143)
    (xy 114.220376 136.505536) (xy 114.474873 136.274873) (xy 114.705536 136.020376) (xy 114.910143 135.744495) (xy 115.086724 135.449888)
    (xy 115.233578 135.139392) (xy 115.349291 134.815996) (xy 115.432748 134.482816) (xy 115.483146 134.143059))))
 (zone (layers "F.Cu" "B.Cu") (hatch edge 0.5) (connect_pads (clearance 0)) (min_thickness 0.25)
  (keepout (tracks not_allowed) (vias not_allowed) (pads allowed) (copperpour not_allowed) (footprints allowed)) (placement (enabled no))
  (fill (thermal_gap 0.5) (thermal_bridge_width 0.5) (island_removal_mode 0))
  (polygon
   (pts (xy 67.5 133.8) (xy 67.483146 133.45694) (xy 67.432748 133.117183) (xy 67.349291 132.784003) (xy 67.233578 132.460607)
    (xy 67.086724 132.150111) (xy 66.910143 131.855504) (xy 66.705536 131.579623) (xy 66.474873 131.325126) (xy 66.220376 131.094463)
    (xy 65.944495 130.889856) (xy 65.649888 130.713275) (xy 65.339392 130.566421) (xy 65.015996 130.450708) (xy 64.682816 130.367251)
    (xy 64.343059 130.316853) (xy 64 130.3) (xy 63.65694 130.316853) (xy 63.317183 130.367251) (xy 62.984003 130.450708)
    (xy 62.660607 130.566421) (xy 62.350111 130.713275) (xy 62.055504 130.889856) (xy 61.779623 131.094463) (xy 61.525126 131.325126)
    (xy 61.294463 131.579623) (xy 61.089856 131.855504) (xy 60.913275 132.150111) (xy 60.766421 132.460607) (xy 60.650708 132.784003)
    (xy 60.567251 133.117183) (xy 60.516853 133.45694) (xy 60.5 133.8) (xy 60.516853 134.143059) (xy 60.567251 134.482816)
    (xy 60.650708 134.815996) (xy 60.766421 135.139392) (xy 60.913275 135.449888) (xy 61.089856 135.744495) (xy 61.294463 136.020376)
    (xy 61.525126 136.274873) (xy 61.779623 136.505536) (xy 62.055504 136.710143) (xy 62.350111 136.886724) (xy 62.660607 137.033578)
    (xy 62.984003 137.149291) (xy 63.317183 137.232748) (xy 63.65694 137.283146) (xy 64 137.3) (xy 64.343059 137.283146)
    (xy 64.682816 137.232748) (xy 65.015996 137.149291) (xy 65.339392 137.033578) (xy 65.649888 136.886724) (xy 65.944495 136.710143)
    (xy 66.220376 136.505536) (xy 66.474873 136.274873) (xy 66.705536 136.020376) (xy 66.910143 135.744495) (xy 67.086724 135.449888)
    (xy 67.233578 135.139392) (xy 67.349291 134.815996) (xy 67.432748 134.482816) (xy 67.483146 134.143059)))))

